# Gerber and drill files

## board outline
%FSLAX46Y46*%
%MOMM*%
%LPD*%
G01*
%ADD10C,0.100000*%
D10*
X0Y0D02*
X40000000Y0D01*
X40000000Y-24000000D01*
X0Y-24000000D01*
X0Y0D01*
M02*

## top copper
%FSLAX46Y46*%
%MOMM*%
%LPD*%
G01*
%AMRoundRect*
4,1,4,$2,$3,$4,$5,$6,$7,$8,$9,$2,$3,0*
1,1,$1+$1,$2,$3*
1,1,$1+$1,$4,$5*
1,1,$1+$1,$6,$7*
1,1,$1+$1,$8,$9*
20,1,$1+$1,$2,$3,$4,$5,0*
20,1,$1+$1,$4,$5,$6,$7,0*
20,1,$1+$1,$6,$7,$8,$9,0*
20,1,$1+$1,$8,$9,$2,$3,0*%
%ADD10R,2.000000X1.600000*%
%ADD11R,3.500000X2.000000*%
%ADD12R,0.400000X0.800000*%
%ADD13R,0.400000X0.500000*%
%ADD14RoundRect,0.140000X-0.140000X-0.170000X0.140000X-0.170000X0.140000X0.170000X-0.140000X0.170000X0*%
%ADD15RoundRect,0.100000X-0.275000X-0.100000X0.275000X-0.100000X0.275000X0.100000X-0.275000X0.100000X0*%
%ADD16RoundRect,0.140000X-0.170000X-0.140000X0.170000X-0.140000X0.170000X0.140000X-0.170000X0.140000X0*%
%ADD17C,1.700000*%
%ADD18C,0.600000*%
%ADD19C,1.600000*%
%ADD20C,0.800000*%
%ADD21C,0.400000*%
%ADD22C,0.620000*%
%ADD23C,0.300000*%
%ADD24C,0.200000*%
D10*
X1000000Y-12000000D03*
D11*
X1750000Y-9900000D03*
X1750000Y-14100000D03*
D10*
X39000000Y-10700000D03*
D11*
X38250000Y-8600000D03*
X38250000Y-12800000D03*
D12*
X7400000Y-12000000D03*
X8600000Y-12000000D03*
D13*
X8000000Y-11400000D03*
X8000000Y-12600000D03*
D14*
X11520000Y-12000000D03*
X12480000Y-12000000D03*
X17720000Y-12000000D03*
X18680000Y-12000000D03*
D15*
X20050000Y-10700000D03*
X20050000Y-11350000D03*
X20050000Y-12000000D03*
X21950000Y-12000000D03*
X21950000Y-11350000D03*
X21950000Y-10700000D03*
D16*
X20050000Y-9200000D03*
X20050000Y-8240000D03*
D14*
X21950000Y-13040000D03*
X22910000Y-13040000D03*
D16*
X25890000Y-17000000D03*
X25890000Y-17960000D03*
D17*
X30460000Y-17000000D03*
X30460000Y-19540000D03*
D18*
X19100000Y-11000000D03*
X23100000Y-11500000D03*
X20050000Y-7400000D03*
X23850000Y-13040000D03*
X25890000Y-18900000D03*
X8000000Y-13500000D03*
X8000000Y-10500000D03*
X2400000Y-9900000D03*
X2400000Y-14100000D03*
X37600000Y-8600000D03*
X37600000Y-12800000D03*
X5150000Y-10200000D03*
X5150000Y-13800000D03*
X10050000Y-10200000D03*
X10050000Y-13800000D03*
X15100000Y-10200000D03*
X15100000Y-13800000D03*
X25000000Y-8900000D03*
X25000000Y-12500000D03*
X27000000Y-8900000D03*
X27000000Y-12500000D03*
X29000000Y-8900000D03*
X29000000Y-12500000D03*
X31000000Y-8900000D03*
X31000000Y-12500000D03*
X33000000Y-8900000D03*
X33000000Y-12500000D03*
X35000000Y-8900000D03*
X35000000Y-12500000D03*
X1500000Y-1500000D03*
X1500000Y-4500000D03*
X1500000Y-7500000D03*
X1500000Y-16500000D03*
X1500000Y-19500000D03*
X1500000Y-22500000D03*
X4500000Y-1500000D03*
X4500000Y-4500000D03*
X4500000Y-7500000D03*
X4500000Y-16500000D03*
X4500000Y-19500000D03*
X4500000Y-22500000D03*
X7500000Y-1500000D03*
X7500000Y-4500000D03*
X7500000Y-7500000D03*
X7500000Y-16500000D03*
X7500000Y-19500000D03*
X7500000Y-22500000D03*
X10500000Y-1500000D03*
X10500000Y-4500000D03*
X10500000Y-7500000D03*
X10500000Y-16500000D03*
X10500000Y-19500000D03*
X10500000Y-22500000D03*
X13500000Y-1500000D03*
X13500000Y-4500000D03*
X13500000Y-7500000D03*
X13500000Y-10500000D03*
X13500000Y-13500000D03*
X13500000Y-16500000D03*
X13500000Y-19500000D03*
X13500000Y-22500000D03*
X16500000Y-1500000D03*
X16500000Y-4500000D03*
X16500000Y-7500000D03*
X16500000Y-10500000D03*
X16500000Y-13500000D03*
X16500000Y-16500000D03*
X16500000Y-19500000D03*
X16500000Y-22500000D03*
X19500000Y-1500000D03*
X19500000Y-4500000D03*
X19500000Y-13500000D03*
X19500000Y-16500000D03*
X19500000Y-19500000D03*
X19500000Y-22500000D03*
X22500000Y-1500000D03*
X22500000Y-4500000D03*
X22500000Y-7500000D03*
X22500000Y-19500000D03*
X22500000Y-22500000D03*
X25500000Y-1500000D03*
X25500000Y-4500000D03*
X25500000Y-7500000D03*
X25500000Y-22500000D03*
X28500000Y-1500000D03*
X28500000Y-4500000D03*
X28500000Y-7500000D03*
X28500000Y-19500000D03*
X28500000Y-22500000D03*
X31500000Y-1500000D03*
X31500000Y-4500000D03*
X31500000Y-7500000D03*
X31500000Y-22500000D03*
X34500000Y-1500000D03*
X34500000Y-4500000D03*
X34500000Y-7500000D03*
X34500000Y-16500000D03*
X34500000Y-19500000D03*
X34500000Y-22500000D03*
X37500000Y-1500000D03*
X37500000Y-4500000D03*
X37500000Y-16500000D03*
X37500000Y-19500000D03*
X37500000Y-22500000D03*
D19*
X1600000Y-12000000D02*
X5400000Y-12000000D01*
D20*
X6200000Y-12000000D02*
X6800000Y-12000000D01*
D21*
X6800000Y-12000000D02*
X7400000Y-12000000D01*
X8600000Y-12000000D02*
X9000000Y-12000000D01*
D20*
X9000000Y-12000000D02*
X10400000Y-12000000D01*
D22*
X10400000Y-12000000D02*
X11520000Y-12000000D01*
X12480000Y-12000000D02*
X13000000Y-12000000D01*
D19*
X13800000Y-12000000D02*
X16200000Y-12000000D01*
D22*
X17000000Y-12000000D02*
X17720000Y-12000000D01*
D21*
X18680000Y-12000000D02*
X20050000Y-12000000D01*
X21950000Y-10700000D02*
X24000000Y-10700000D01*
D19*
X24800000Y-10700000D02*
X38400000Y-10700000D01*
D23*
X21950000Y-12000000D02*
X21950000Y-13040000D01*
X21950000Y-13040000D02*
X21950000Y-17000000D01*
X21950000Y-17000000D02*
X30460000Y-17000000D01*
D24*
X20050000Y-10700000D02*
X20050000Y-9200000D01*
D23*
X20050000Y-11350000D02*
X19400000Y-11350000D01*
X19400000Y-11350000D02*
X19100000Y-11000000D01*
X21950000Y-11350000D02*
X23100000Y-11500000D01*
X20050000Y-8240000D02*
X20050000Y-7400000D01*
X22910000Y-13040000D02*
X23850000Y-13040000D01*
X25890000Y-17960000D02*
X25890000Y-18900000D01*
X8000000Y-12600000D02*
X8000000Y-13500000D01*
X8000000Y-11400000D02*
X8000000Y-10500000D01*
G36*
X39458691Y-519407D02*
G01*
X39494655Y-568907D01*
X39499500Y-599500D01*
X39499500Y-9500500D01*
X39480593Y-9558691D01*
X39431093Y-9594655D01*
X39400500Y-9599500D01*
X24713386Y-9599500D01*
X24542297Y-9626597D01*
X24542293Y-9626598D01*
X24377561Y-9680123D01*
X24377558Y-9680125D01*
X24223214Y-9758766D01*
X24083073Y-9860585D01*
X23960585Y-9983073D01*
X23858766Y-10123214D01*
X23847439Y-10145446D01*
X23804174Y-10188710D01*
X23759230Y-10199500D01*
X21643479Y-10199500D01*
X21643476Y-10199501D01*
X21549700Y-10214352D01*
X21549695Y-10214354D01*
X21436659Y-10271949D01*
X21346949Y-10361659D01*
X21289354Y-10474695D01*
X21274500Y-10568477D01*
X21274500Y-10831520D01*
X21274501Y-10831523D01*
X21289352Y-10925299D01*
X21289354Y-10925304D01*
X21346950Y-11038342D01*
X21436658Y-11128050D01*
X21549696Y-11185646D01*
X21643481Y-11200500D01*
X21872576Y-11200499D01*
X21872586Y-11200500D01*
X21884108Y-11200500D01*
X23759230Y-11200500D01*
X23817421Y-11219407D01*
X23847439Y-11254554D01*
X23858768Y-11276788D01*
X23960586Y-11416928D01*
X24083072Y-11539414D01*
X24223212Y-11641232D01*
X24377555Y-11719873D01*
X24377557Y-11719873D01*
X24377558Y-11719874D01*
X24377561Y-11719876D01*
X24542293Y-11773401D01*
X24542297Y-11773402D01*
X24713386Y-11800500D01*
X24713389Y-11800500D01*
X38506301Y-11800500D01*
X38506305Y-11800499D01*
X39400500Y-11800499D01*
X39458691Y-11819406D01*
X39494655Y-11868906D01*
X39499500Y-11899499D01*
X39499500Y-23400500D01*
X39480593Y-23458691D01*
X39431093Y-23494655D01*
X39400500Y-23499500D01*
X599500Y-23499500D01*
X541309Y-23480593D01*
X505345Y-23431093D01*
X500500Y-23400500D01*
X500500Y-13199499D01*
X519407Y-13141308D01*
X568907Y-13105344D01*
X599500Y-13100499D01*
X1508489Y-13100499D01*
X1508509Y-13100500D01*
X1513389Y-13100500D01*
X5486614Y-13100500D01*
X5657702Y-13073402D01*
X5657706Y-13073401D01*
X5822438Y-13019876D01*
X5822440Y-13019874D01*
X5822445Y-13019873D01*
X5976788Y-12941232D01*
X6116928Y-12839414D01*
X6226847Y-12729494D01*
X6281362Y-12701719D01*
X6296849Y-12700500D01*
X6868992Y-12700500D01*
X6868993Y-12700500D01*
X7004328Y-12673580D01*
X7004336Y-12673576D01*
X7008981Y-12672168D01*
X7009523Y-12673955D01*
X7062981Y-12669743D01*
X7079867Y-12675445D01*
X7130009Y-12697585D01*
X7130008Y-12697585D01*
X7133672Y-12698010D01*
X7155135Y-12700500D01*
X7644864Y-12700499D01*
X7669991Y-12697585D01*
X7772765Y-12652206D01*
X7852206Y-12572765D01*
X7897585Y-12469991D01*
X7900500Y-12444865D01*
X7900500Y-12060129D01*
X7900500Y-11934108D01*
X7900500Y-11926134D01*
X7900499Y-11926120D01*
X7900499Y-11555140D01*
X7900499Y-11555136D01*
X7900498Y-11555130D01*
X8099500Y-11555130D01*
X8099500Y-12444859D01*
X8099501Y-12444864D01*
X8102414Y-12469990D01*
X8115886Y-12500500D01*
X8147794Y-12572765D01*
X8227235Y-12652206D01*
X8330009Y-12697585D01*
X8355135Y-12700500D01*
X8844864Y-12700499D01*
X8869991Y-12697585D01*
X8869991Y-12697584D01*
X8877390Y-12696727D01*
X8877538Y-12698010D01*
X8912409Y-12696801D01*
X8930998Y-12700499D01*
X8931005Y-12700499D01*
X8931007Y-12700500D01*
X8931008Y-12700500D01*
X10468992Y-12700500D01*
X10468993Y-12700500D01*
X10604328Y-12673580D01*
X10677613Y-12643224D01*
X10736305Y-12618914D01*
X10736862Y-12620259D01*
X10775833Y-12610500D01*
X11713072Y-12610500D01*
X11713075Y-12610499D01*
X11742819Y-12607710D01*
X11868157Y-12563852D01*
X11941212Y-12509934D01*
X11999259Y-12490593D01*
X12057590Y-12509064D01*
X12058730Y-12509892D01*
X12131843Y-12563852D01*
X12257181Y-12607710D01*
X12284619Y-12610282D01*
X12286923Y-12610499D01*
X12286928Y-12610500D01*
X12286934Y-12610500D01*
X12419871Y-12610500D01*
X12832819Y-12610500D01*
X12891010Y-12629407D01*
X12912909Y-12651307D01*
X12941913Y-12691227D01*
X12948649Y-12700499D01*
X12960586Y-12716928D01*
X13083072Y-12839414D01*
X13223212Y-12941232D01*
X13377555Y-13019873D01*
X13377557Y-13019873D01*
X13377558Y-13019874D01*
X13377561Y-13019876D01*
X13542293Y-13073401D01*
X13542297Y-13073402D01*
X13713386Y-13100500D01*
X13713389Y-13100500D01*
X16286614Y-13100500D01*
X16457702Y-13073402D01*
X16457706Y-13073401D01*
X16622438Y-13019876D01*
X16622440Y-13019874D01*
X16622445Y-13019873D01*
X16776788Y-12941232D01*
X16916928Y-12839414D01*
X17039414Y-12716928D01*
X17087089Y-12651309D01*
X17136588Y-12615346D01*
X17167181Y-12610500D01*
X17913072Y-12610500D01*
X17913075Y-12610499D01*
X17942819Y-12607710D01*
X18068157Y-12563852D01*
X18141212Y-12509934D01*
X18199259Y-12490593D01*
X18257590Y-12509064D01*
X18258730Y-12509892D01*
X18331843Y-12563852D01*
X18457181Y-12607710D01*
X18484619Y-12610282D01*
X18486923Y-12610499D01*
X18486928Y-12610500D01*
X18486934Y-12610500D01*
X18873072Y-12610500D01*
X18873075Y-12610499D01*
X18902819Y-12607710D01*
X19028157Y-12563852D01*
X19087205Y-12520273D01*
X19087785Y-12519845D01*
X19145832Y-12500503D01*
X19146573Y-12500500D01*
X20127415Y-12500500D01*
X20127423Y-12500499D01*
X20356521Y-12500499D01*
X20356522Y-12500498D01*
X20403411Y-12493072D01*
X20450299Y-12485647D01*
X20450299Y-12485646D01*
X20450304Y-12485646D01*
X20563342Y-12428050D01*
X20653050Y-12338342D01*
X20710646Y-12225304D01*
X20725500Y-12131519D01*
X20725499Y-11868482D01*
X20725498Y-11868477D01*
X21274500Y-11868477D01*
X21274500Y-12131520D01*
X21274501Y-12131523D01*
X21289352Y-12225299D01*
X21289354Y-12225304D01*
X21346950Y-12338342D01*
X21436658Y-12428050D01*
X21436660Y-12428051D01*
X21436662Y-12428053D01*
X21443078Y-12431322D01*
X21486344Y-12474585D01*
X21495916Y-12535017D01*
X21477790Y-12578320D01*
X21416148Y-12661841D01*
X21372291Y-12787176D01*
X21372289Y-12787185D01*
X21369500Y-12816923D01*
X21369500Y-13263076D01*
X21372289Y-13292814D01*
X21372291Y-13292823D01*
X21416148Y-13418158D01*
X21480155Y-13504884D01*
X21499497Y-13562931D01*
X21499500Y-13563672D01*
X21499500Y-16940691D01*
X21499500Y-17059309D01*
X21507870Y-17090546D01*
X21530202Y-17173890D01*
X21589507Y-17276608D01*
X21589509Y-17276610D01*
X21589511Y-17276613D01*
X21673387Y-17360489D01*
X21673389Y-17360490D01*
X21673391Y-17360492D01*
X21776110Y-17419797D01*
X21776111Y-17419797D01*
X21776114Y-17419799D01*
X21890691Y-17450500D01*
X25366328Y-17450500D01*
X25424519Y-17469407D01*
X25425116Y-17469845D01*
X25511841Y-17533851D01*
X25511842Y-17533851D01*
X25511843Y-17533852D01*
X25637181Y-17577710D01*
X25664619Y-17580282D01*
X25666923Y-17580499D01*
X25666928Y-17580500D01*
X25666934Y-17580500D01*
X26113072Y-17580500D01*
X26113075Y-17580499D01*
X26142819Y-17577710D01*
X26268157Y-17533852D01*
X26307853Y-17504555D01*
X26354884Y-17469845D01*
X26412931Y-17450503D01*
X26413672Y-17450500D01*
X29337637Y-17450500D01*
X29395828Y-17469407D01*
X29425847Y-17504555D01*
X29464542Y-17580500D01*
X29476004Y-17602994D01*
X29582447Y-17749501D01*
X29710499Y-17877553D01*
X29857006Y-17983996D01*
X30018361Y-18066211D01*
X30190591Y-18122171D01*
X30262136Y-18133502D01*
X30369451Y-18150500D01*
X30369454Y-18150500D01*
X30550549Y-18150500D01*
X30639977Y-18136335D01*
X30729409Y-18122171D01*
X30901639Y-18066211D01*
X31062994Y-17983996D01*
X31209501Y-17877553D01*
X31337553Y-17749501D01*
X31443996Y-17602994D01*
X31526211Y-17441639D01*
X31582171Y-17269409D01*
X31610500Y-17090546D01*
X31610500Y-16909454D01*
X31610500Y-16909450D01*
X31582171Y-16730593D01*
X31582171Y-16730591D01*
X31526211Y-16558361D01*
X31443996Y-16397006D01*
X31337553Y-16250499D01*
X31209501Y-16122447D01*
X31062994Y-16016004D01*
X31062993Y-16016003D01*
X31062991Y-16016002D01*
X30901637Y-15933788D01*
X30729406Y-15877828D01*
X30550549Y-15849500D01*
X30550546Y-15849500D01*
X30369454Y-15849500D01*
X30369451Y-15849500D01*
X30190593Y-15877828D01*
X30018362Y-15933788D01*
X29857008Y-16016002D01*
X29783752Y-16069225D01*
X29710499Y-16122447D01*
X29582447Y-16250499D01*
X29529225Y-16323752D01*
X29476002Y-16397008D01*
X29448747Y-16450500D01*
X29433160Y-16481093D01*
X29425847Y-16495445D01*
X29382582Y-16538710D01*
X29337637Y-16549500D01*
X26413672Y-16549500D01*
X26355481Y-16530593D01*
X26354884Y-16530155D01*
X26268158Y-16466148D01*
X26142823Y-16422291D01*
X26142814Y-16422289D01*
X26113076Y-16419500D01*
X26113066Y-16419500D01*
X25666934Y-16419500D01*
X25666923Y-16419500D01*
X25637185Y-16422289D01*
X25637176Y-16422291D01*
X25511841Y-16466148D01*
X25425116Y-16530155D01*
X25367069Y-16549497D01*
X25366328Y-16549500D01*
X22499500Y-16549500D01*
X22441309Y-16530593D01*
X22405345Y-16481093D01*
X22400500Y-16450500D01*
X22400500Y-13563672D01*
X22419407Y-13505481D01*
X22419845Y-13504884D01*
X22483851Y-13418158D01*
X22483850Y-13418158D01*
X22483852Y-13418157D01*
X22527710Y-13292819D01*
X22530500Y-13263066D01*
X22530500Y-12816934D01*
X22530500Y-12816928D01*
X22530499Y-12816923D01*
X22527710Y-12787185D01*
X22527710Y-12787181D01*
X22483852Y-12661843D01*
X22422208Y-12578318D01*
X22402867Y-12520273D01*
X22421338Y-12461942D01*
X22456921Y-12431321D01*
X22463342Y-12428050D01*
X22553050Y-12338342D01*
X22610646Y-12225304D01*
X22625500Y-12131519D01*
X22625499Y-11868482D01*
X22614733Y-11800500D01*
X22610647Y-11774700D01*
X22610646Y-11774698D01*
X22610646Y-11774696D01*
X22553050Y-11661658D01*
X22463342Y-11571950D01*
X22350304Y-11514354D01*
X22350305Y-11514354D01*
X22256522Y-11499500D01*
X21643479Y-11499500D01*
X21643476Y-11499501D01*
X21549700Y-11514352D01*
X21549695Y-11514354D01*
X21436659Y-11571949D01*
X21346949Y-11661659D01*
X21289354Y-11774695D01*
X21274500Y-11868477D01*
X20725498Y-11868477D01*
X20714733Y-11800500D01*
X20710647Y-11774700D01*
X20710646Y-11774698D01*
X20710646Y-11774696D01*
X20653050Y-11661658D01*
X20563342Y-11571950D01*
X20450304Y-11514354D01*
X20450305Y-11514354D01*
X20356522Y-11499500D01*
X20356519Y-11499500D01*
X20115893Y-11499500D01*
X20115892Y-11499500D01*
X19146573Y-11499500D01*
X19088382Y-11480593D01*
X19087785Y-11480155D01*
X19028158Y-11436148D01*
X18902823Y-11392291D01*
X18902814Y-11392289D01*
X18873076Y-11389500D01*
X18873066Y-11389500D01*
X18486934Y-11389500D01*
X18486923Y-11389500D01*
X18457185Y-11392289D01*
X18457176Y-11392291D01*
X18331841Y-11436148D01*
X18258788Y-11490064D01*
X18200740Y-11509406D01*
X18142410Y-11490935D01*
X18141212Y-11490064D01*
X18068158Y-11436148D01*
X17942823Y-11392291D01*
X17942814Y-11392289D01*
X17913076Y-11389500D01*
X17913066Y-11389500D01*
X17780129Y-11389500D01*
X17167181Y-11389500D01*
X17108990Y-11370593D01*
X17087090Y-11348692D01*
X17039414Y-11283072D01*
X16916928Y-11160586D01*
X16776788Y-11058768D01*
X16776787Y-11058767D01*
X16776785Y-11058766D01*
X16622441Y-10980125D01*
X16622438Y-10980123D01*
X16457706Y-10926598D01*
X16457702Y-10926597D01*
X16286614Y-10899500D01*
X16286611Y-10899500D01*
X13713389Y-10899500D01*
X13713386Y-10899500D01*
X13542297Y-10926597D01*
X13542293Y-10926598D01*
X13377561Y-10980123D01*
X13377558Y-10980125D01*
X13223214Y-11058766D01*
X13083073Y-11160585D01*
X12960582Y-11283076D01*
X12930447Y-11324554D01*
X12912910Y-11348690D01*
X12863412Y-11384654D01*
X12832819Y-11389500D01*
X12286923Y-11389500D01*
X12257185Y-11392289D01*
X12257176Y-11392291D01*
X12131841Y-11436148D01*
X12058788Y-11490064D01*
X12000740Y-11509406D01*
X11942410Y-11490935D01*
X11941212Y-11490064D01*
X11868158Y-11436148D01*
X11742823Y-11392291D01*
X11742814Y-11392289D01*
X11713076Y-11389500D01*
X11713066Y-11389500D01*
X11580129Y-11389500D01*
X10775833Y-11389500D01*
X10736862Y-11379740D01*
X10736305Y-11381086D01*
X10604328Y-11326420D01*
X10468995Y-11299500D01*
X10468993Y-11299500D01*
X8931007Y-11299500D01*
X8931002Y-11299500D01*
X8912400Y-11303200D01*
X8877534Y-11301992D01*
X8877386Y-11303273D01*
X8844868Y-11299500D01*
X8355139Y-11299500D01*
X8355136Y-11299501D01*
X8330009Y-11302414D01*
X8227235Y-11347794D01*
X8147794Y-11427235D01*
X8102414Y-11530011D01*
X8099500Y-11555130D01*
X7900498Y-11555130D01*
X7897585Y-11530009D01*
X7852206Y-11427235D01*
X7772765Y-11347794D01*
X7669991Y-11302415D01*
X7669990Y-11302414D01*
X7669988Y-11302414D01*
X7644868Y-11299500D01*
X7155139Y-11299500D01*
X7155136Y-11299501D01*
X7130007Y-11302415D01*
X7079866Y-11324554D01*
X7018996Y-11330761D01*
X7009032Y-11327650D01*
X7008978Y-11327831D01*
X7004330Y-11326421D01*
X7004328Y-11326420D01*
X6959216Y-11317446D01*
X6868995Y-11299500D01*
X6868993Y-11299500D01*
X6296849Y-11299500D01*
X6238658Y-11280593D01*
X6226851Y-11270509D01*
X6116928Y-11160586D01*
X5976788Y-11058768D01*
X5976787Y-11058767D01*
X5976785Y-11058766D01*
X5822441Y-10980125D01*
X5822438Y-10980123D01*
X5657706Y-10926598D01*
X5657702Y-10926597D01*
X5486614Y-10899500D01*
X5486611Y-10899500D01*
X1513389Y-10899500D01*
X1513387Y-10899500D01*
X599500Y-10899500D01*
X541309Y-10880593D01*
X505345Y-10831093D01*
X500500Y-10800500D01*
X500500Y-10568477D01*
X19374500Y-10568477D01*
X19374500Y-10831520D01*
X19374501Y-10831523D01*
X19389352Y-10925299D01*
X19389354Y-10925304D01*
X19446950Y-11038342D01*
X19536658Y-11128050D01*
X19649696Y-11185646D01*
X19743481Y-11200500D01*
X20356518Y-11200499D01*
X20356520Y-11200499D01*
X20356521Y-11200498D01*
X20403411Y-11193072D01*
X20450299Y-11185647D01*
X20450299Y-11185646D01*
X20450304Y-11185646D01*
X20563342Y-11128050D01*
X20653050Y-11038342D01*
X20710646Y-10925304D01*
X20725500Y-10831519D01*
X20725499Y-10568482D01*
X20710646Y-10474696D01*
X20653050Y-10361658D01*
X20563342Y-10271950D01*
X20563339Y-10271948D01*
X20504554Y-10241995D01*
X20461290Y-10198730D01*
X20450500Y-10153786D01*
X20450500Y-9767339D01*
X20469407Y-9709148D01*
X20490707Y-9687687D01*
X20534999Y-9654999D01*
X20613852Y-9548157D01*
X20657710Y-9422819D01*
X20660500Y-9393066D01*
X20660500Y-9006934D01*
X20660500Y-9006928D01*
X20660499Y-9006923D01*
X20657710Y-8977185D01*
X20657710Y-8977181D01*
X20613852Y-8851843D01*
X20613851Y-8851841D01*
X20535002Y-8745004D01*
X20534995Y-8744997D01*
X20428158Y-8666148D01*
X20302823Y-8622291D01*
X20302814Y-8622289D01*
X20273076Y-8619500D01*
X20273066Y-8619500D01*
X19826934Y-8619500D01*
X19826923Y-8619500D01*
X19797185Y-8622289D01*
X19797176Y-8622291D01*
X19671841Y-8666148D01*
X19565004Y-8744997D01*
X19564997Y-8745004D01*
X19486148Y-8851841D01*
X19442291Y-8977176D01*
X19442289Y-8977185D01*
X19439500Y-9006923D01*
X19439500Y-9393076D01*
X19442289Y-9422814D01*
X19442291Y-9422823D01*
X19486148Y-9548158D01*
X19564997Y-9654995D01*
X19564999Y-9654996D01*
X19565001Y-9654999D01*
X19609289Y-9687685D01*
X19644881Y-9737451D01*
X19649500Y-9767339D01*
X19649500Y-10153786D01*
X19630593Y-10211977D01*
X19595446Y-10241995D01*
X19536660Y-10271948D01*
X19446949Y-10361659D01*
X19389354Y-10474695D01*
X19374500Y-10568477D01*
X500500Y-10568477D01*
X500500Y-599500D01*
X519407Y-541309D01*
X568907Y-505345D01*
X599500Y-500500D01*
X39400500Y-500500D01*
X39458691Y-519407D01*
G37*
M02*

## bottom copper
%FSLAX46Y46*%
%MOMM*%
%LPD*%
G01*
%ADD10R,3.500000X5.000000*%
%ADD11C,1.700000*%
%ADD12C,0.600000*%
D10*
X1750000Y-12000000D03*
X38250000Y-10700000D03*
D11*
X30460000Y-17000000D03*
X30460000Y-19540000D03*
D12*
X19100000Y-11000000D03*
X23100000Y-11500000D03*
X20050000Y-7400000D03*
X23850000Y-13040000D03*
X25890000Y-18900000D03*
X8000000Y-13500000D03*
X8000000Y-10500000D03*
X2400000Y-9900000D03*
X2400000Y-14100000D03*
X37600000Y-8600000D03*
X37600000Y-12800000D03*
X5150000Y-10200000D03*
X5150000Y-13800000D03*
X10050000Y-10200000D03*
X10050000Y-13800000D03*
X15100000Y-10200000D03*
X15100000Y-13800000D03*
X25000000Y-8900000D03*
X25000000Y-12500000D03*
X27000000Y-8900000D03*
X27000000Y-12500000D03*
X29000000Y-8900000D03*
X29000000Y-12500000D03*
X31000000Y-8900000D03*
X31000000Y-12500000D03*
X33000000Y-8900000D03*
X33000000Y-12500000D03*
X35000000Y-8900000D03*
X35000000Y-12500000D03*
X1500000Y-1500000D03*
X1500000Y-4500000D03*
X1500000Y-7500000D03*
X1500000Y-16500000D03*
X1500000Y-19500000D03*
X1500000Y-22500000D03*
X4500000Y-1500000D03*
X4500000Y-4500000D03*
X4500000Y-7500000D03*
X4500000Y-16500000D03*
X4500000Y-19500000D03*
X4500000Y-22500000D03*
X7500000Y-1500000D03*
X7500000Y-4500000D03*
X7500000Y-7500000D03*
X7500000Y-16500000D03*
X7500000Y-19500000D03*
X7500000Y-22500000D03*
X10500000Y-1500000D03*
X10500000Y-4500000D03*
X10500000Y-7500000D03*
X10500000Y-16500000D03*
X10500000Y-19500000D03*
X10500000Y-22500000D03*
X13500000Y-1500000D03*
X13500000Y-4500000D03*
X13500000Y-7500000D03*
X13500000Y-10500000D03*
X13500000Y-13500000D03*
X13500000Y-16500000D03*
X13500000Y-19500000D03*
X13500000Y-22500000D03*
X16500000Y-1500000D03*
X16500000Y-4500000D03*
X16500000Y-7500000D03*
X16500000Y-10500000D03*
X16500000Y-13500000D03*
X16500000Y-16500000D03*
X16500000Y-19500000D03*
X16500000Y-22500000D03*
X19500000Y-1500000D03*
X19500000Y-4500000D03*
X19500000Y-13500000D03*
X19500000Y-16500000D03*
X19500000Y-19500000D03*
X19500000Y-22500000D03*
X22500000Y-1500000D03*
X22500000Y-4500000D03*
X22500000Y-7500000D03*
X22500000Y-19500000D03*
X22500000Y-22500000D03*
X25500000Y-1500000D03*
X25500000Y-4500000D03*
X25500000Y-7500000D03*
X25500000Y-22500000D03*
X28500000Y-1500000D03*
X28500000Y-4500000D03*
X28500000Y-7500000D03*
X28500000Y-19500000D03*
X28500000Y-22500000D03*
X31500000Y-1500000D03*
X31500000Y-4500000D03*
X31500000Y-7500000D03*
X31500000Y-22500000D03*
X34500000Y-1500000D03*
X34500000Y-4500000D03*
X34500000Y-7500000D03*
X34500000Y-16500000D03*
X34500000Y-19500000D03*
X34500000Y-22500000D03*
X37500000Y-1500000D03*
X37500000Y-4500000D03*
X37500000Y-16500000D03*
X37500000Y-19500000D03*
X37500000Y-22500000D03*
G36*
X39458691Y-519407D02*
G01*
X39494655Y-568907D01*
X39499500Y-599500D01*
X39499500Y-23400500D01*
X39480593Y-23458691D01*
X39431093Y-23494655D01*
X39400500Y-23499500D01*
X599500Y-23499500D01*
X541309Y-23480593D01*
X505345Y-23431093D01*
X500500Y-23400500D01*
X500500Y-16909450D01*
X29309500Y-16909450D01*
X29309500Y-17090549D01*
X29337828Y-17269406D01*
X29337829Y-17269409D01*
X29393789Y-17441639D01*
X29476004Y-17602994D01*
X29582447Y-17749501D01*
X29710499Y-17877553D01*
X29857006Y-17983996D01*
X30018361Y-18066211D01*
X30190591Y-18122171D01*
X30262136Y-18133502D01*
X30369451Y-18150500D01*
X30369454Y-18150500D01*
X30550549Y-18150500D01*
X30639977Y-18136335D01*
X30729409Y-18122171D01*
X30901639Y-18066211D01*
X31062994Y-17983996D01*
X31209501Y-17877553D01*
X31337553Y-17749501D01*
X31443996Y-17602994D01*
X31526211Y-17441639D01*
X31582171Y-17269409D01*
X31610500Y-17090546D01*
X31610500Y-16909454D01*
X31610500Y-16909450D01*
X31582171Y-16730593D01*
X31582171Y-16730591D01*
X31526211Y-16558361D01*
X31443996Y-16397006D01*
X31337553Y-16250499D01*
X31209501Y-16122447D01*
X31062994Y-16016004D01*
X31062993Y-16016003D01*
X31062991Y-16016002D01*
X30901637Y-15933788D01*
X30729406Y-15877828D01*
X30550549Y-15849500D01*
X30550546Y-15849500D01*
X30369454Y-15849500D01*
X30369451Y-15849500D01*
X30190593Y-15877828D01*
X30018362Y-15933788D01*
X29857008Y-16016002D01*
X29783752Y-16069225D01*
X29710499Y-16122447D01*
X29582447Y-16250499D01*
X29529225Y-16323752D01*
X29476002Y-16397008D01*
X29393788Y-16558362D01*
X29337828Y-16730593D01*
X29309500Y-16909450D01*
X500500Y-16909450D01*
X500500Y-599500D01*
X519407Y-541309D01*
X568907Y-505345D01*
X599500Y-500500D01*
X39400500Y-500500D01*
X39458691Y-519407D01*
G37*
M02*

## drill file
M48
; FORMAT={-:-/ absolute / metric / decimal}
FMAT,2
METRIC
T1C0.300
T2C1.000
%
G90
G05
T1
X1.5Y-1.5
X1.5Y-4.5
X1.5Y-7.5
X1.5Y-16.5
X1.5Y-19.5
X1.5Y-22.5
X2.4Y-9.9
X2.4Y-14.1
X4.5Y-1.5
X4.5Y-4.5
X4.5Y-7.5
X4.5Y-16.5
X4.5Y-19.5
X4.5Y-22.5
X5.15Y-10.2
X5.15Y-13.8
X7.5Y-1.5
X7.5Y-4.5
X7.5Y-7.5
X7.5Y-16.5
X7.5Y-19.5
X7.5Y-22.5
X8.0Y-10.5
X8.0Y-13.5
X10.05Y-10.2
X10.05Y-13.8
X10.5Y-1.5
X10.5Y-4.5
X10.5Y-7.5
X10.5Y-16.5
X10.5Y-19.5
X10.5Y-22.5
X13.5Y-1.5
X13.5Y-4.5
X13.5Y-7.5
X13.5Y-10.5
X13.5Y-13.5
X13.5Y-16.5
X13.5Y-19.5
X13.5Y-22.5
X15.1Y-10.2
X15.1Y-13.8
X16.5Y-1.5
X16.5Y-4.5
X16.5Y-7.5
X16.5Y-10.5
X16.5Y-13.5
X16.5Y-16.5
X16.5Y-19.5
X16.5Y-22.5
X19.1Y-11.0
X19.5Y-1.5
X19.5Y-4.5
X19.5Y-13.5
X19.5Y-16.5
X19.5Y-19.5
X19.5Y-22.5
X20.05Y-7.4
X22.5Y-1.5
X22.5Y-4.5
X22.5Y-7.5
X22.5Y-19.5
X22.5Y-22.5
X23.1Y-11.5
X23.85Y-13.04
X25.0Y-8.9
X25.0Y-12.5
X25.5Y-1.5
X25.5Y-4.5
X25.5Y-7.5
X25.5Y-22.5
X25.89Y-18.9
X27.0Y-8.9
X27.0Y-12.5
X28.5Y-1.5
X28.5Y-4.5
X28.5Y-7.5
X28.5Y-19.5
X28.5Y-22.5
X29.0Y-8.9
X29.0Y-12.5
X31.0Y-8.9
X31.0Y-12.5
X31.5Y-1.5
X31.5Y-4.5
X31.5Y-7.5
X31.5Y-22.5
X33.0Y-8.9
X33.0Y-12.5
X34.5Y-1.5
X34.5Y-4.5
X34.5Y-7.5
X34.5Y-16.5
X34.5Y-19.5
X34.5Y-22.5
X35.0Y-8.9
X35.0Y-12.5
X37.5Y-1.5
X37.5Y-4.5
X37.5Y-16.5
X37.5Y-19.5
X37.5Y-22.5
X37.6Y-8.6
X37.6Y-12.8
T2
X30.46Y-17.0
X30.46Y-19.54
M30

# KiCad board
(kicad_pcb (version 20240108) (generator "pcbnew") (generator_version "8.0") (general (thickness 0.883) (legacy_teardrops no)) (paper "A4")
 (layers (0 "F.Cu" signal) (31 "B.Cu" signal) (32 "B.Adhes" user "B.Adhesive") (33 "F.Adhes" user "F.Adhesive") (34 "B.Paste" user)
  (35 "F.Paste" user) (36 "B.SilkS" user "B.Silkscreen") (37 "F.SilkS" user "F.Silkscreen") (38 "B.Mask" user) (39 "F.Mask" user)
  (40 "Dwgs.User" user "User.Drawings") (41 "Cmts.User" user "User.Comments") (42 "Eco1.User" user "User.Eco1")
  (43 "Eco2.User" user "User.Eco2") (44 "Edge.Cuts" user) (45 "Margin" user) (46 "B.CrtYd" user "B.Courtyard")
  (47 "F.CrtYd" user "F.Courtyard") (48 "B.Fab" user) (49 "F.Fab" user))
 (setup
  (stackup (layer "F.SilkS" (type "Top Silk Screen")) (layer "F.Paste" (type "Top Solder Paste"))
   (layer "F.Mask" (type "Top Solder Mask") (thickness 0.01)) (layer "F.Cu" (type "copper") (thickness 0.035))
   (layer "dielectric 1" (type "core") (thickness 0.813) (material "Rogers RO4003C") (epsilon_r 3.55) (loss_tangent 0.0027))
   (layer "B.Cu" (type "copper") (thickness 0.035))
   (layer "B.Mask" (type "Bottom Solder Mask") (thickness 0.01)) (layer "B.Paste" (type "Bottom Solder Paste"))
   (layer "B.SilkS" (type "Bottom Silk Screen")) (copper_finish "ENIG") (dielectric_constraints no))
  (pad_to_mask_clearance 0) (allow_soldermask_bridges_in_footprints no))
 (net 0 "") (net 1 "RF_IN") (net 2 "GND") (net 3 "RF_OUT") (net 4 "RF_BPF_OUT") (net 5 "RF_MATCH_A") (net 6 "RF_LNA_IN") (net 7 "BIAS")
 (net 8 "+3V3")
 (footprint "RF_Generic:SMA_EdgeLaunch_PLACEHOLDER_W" (layer "F.Cu") (at 0 12)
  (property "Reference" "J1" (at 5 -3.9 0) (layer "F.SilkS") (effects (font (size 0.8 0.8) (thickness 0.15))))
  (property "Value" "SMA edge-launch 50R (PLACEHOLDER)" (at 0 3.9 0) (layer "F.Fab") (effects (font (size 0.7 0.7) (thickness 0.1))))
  (pad "1" smd rect (at 1 0) (size 2 1.6) (layers "F.Cu" "F.Paste" "F.Mask") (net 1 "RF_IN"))
  (pad "2" smd rect (at 1.75 -2.1) (size 3.5 2) (layers "F.Cu" "F.Paste" "F.Mask") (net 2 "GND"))
  (pad "3" smd rect (at 1.75 2.1) (size 3.5 2) (layers "F.Cu" "F.Paste" "F.Mask") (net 2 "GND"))
  (pad "4" smd rect (at 1.75 0) (size 3.5 5) (layers "B.Cu" "B.Paste" "B.Mask") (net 2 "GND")))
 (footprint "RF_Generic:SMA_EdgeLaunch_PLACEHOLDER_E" (layer "F.Cu") (at 40 10.7)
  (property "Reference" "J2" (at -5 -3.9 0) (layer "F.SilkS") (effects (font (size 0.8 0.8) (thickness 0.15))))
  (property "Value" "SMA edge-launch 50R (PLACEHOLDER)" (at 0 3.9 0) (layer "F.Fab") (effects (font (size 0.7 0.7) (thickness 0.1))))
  (pad "1" smd rect (at -1 0) (size 2 1.6) (layers "F.Cu" "F.Paste" "F.Mask") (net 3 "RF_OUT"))
  (pad "2" smd rect (at -1.75 -2.1) (size 3.5 2) (layers "F.Cu" "F.Paste" "F.Mask") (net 2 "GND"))
  (pad "3" smd rect (at -1.75 2.1) (size 3.5 2) (layers "F.Cu" "F.Paste" "F.Mask") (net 2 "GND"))
  (pad "4" smd rect (at -1.75 0) (size 3.5 5) (layers "B.Cu" "B.Paste" "B.Mask") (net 2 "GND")))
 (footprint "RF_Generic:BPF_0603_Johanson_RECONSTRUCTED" (layer "F.Cu") (at 8 12)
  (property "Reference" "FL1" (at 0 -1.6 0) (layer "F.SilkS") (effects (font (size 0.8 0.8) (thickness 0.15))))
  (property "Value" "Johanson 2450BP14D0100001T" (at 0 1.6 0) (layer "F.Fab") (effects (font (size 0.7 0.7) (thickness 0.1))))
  (pad "2" smd rect (at -0.6 0) (size 0.4 0.8) (layers "F.Cu" "F.Paste" "F.Mask") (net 1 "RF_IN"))
  (pad "4" smd rect (at 0.6 0) (size 0.4 0.8) (layers "F.Cu" "F.Paste" "F.Mask") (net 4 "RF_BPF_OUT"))
  (pad "1" smd rect (at 0 -0.6) (size 0.4 0.5) (layers "F.Cu" "F.Paste" "F.Mask") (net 2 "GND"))
  (pad "3" smd rect (at 0 0.6) (size 0.4 0.5) (layers "F.Cu" "F.Paste" "F.Mask") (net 2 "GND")))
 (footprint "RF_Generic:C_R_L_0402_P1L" (layer "F.Cu") (at 12 12)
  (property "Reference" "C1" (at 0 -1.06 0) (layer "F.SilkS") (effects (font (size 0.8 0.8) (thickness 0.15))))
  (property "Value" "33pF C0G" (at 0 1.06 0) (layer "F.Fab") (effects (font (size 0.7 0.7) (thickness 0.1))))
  (pad "1" smd roundrect (at -0.48 0) (size 0.56 0.62) (layers "F.Cu" "F.Paste" "F.Mask") (roundrect_rratio 0.25) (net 4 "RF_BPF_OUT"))
  (pad "2" smd roundrect (at 0.48 0) (size 0.56 0.62) (layers "F.Cu" "F.Paste" "F.Mask") (roundrect_rratio 0.25) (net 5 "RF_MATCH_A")))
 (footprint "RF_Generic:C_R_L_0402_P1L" (layer "F.Cu") (at 18.2 12)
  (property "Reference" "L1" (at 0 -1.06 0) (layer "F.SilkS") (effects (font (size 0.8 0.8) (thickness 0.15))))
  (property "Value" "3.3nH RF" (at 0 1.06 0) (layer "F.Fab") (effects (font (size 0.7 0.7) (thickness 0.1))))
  (pad "1" smd roundrect (at -0.48 0) (size 0.56 0.62) (layers "F.Cu" "F.Paste" "F.Mask") (roundrect_rratio 0.25) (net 5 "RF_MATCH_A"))
  (pad "2" smd roundrect (at 0.48 0) (size 0.56 0.62) (layers "F.Cu" "F.Paste" "F.Mask") (roundrect_rratio 0.25) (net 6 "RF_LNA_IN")))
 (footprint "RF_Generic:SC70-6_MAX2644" (layer "F.Cu") (at 21 11.35)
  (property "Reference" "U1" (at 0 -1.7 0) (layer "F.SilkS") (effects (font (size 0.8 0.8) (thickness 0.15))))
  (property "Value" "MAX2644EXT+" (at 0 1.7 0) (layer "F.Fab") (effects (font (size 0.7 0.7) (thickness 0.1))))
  (pad "1" smd roundrect (at -0.95 -0.65) (size 0.75 0.4) (layers "F.Cu" "F.Paste" "F.Mask") (roundrect_rratio 0.25) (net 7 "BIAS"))
  (pad "2" smd roundrect (at -0.95 0) (size 0.75 0.4) (layers "F.Cu" "F.Paste" "F.Mask") (roundrect_rratio 0.25) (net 2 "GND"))
  (pad "3" smd roundrect (at -0.95 0.65) (size 0.75 0.4) (layers "F.Cu" "F.Paste" "F.Mask") (roundrect_rratio 0.25) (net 6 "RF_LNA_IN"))
  (pad "4" smd roundrect (at 0.95 0.65) (size 0.75 0.4) (layers "F.Cu" "F.Paste" "F.Mask") (roundrect_rratio 0.25) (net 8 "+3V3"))
  (pad "5" smd roundrect (at 0.95 0) (size 0.75 0.4) (layers "F.Cu" "F.Paste" "F.Mask") (roundrect_rratio 0.25) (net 2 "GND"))
  (pad "6" smd roundrect (at 0.95 -0.65) (size 0.75 0.4) (layers "F.Cu" "F.Paste" "F.Mask") (roundrect_rratio 0.25) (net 3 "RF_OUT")))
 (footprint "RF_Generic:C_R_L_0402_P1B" (layer "F.Cu") (at 20.05 8.72)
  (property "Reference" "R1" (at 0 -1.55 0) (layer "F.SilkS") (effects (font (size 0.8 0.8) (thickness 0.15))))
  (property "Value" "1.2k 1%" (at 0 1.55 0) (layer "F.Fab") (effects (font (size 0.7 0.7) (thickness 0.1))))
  (pad "1" smd roundrect (at 0 0.48) (size 0.62 0.56) (layers "F.Cu" "F.Paste" "F.Mask") (roundrect_rratio 0.25) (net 7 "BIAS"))
  (pad "2" smd roundrect (at 0 -0.48) (size 0.62 0.56) (layers "F.Cu" "F.Paste" "F.Mask") (roundrect_rratio 0.25) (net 2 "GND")))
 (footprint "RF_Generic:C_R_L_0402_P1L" (layer "F.Cu") (at 22.43 13.04)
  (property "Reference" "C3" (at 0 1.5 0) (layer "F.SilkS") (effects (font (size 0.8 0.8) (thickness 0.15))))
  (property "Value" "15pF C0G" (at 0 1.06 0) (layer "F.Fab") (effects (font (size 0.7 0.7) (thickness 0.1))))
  (pad "1" smd roundrect (at -0.48 0) (size 0.56 0.62) (layers "F.Cu" "F.Paste" "F.Mask") (roundrect_rratio 0.25) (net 8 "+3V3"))
  (pad "2" smd roundrect (at 0.48 0) (size 0.56 0.62) (layers "F.Cu" "F.Paste" "F.Mask") (roundrect_rratio 0.25) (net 2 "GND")))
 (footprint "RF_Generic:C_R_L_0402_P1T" (layer "F.Cu") (at 25.89 17.48)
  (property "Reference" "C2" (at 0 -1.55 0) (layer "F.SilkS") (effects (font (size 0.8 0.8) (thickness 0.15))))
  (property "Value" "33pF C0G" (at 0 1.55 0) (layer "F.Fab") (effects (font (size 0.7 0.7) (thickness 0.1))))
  (pad "1" smd roundrect (at 0 -0.48) (size 0.62 0.56) (layers "F.Cu" "F.Paste" "F.Mask") (roundrect_rratio 0.25) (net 8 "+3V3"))
  (pad "2" smd roundrect (at 0 0.48) (size 0.62 0.56) (layers "F.Cu" "F.Paste" "F.Mask") (roundrect_rratio 0.25) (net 2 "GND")))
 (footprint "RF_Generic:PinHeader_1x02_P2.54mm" (layer "F.Cu") (at 30.46 17)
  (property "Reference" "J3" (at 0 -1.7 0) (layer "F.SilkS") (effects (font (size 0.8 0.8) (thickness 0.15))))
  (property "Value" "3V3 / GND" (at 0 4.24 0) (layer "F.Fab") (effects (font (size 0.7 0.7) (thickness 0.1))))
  (pad "1" thru_hole circle (at 0 0) (size 1.7 1.7) (drill 1) (layers "*.Cu" "*.Mask") (remove_unused_layers no) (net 8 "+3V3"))
  (pad "2" thru_hole circle (at 0 2.54) (size 1.7 1.7) (drill 1) (layers "*.Cu" "*.Mask") (remove_unused_layers no) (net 2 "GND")))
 (segment (start 1.6 12) (end 5.4 12) (width 1.6) (layer "F.Cu") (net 1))
 (segment (start 6.2 12) (end 6.8 12) (width 0.8) (layer "F.Cu") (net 1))
 (segment (start 6.8 12) (end 7.4 12) (width 0.4) (layer "F.Cu") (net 1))
 (segment (start 8.6 12) (end 9 12) (width 0.4) (layer "F.Cu") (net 4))
 (segment (start 9 12) (end 10.4 12) (width 0.8) (layer "F.Cu") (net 4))
 (segment (start 10.4 12) (end 11.52 12) (width 0.62) (layer "F.Cu") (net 4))
 (segment (start 12.48 12) (end 13 12) (width 0.62) (layer "F.Cu") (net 5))
 (segment (start 13.8 12) (end 16.2 12) (width 1.6) (layer "F.Cu") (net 5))
 (segment (start 17 12) (end 17.72 12) (width 0.62) (layer "F.Cu") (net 5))
 (segment (start 18.68 12) (end 20.05 12) (width 0.4) (layer "F.Cu") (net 6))
 (segment (start 21.95 10.7) (end 24 10.7) (width 0.4) (layer "F.Cu") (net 3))
 (segment (start 24.8 10.7) (end 38.4 10.7) (width 1.6) (layer "F.Cu") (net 3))
 (segment (start 21.95 12) (end 21.95 13.04) (width 0.3) (layer "F.Cu") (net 8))
 (segment (start 21.95 13.04) (end 21.95 17) (width 0.3) (layer "F.Cu") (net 8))
 (segment (start 21.95 17) (end 30.46 17) (width 0.3) (layer "F.Cu") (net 8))
 (segment (start 20.05 10.7) (end 20.05 9.2) (width 0.2) (layer "F.Cu") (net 7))
 (segment (start 20.05 11.35) (end 19.4 11.35) (width 0.3) (layer "F.Cu") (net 2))
 (segment (start 19.4 11.35) (end 19.1 11) (width 0.3) (layer "F.Cu") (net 2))
 (segment (start 21.95 11.35) (end 23.1 11.5) (width 0.3) (layer "F.Cu") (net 2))
 (segment (start 20.05 8.24) (end 20.05 7.4) (width 0.3) (layer "F.Cu") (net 2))
 (segment (start 22.91 13.04) (end 23.85 13.04) (width 0.3) (layer "F.Cu") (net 2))
 (segment (start 25.89 17.96) (end 25.89 18.9) (width 0.3) (layer "F.Cu") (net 2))
 (segment (start 8 12.6) (end 8 13.5) (width 0.3) (layer "F.Cu") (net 2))
 (segment (start 8 11.4) (end 8 10.5) (width 0.3) (layer "F.Cu") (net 2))
 (via (at 19.1 11) (size 0.6) (drill 0.3) (layers "F.Cu" "B.Cu") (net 2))
 (via (at 23.1 11.5) (size 0.6) (drill 0.3) (layers "F.Cu" "B.Cu") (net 2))
 (via (at 20.05 7.4) (size 0.6) (drill 0.3) (layers "F.Cu" "B.Cu") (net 2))
 (via (at 23.85 13.04) (size 0.6) (drill 0.3) (layers "F.Cu" "B.Cu") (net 2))
 (via (at 25.89 18.9) (size 0.6) (drill 0.3) (layers "F.Cu" "B.Cu") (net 2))
 (via (at 8 13.5) (size 0.6) (drill 0.3) (layers "F.Cu" "B.Cu") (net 2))
 (via (at 8 10.5) (size 0.6) (drill 0.3) (layers "F.Cu" "B.Cu") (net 2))
 (via (at 2.4 9.9) (size 0.6) (drill 0.3) (layers "F.Cu" "B.Cu") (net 2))
 (via (at 2.4 14.1) (size 0.6) (drill 0.3) (layers "F.Cu" "B.Cu") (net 2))
 (via (at 37.6 8.6) (size 0.6) (drill 0.3) (layers "F.Cu" "B.Cu") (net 2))
 (via (at 37.6 12.8) (size 0.6) (drill 0.3) (layers "F.Cu" "B.Cu") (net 2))
 (via (at 5.15 10.2) (size 0.6) (drill 0.3) (layers "F.Cu" "B.Cu") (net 2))
 (via (at 5.15 13.8) (size 0.6) (drill 0.3) (layers "F.Cu" "B.Cu") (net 2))
 (via (at 10.05 10.2) (size 0.6) (drill 0.3) (layers "F.Cu" "B.Cu") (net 2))
 (via (at 10.05 13.8) (size 0.6) (drill 0.3) (layers "F.Cu" "B.Cu") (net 2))
 (via (at 15.1 10.2) (size 0.6) (drill 0.3) (layers "F.Cu" "B.Cu") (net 2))
 (via (at 15.1 13.8) (size 0.6) (drill 0.3) (layers "F.Cu" "B.Cu") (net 2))
 (via (at 25 8.9) (size 0.6) (drill 0.3) (layers "F.Cu" "B.Cu") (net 2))
 (via (at 25 12.5) (size 0.6) (drill 0.3) (layers "F.Cu" "B.Cu") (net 2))
 (via (at 27 8.9) (size 0.6) (drill 0.3) (layers "F.Cu" "B.Cu") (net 2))
 (via (at 27 12.5) (size 0.6) (drill 0.3) (layers "F.Cu" "B.Cu") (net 2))
 (via (at 29 8.9) (size 0.6) (drill 0.3) (layers "F.Cu" "B.Cu") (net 2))
 (via (at 29 12.5) (size 0.6) (drill 0.3) (layers "F.Cu" "B.Cu") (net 2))
 (via (at 31 8.9) (size 0.6) (drill 0.3) (layers "F.Cu" "B.Cu") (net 2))
 (via (at 31 12.5) (size 0.6) (drill 0.3) (layers "F.Cu" "B.Cu") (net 2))
 (via (at 33 8.9) (size 0.6) (drill 0.3) (layers "F.Cu" "B.Cu") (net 2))
 (via (at 33 12.5) (size 0.6) (drill 0.3) (layers "F.Cu" "B.Cu") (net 2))
 (via (at 35 8.9) (size 0.6) (drill 0.3) (layers "F.Cu" "B.Cu") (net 2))
 (via (at 35 12.5) (size 0.6) (drill 0.3) (layers "F.Cu" "B.Cu") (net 2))
 (via (at 1.5 1.5) (size 0.6) (drill 0.3) (layers "F.Cu" "B.Cu") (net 2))
 (via (at 1.5 4.5) (size 0.6) (drill 0.3) (layers "F.Cu" "B.Cu") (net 2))
 (via (at 1.5 7.5) (size 0.6) (drill 0.3) (layers "F.Cu" "B.Cu") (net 2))
 (via (at 1.5 16.5) (size 0.6) (drill 0.3) (layers "F.Cu" "B.Cu") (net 2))
 (via (at 1.5 19.5) (size 0.6) (drill 0.3) (layers "F.Cu" "B.Cu") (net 2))
 (via (at 1.5 22.5) (size 0.6) (drill 0.3) (layers "F.Cu" "B.Cu") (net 2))
 (via (at 4.5 1.5) (size 0.6) (drill 0.3) (layers "F.Cu" "B.Cu") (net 2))
 (via (at 4.5 4.5) (size 0.6) (drill 0.3) (layers "F.Cu" "B.Cu") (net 2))
 (via (at 4.5 7.5) (size 0.6) (drill 0.3) (layers "F.Cu" "B.Cu") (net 2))
 (via (at 4.5 16.5) (size 0.6) (drill 0.3) (layers "F.Cu" "B.Cu") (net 2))
 (via (at 4.5 19.5) (size 0.6) (drill 0.3) (layers "F.Cu" "B.Cu") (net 2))
 (via (at 4.5 22.5) (size 0.6) (drill 0.3) (layers "F.Cu" "B.Cu") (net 2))
 (via (at 7.5 1.5) (size 0.6) (drill 0.3) (layers "F.Cu" "B.Cu") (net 2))
 (via (at 7.5 4.5) (size 0.6) (drill 0.3) (layers "F.Cu" "B.Cu") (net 2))
 (via (at 7.5 7.5) (size 0.6) (drill 0.3) (layers "F.Cu" "B.Cu") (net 2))
 (via (at 7.5 16.5) (size 0.6) (drill 0.3) (layers "F.Cu" "B.Cu") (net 2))
 (via (at 7.5 19.5) (size 0.6) (drill 0.3) (layers "F.Cu" "B.Cu") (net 2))
 (via (at 7.5 22.5) (size 0.6) (drill 0.3) (layers "F.Cu" "B.Cu") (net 2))
 (via (at 10.5 1.5) (size 0.6) (drill 0.3) (layers "F.Cu" "B.Cu") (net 2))
 (via (at 10.5 4.5) (size 0.6) (drill 0.3) (layers "F.Cu" "B.Cu") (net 2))
 (via (at 10.5 7.5) (size 0.6) (drill 0.3) (layers "F.Cu" "B.Cu") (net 2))
 (via (at 10.5 16.5) (size 0.6) (drill 0.3) (layers "F.Cu" "B.Cu") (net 2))
 (via (at 10.5 19.5) (size 0.6) (drill 0.3) (layers "F.Cu" "B.Cu") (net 2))
 (via (at 10.5 22.5) (size 0.6) (drill 0.3) (layers "F.Cu" "B.Cu") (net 2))
 (via (at 13.5 1.5) (size 0.6) (drill 0.3) (layers "F.Cu" "B.Cu") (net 2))
 (via (at 13.5 4.5) (size 0.6) (drill 0.3) (layers "F.Cu" "B.Cu") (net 2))
 (via (at 13.5 7.5) (size 0.6) (drill 0.3) (layers "F.Cu" "B.Cu") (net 2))
 (via (at 13.5 10.5) (size 0.6) (drill 0.3) (layers "F.Cu" "B.Cu") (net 2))
 (via (at 13.5 13.5) (size 0.6) (drill 0.3) (layers "F.Cu" "B.Cu") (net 2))
 (via (at 13.5 16.5) (size 0.6) (drill 0.3) (layers "F.Cu" "B.Cu") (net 2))
 (via (at 13.5 19.5) (size 0.6) (drill 0.3) (layers "F.Cu" "B.Cu") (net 2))
 (via (at 13.5 22.5) (size 0.6) (drill 0.3) (layers "F.Cu" "B.Cu") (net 2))
 (via (at 16.5 1.5) (size 0.6) (drill 0.3) (layers "F.Cu" "B.Cu") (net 2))
 (via (at 16.5 4.5) (size 0.6) (drill 0.3) (layers "F.Cu" "B.Cu") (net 2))
 (via (at 16.5 7.5) (size 0.6) (drill 0.3) (layers "F.Cu" "B.Cu") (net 2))
 (via (at 16.5 10.5) (size 0.6) (drill 0.3) (layers "F.Cu" "B.Cu") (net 2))
 (via (at 16.5 13.5) (size 0.6) (drill 0.3) (layers "F.Cu" "B.Cu") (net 2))
 (via (at 16.5 16.5) (size 0.6) (drill 0.3) (layers "F.Cu" "B.Cu") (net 2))
 (via (at 16.5 19.5) (size 0.6) (drill 0.3) (layers "F.Cu" "B.Cu") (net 2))
 (via (at 16.5 22.5) (size 0.6) (drill 0.3) (layers "F.Cu" "B.Cu") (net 2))
 (via (at 19.5 1.5) (size 0.6) (drill 0.3) (layers "F.Cu" "B.Cu") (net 2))
 (via (at 19.5 4.5) (size 0.6) (drill 0.3) (layers "F.Cu" "B.Cu") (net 2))
 (via (at 19.5 13.5) (size 0.6) (drill 0.3) (layers "F.Cu" "B.Cu") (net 2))
 (via (at 19.5 16.5) (size 0.6) (drill 0.3) (layers "F.Cu" "B.Cu") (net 2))
 (via (at 19.5 19.5) (size 0.6) (drill 0.3) (layers "F.Cu" "B.Cu") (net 2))
 (via (at 19.5 22.5) (size 0.6) (drill 0.3) (layers "F.Cu" "B.Cu") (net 2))
 (via (at 22.5 1.5) (size 0.6) (drill 0.3) (layers "F.Cu" "B.Cu") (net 2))
 (via (at 22.5 4.5) (size 0.6) (drill 0.3) (layers "F.Cu" "B.Cu") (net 2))
 (via (at 22.5 7.5) (size 0.6) (drill 0.3) (layers "F.Cu" "B.Cu") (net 2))
 (via (at 22.5 19.5) (size 0.6) (drill 0.3) (layers "F.Cu" "B.Cu") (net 2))
 (via (at 22.5 22.5) (size 0.6) (drill 0.3) (layers "F.Cu" "B.Cu") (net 2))
 (via (at 25.5 1.5) (size 0.6) (drill 0.3) (layers "F.Cu" "B.Cu") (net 2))
 (via (at 25.5 4.5) (size 0.6) (drill 0.3) (layers "F.Cu" "B.Cu") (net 2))
 (via (at 25.5 7.5) (size 0.6) (drill 0.3) (layers "F.Cu" "B.Cu") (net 2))
 (via (at 25.5 22.5) (size 0.6) (drill 0.3) (layers "F.Cu" "B.Cu") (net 2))
 (via (at 28.5 1.5) (size 0.6) (drill 0.3) (layers "F.Cu" "B.Cu") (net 2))
 (via (at 28.5 4.5) (size 0.6) (drill 0.3) (layers "F.Cu" "B.Cu") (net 2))
 (via (at 28.5 7.5) (size 0.6) (drill 0.3) (layers "F.Cu" "B.Cu") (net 2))
 (via (at 28.5 19.5) (size 0.6) (drill 0.3) (layers "F.Cu" "B.Cu") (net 2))
 (via (at 28.5 22.5) (size 0.6) (drill 0.3) (layers "F.Cu" "B.Cu") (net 2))
 (via (at 31.5 1.5) (size 0.6) (drill 0.3) (layers "F.Cu" "B.Cu") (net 2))
 (via (at 31.5 4.5) (size 0.6) (drill 0.3) (layers "F.Cu" "B.Cu") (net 2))
 (via (at 31.5 7.5) (size 0.6) (drill 0.3) (layers "F.Cu" "B.Cu") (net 2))
 (via (at 31.5 22.5) (size 0.6) (drill 0.3) (layers "F.Cu" "B.Cu") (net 2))
 (via (at 34.5 1.5) (size 0.6) (drill 0.3) (layers "F.Cu" "B.Cu") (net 2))
 (via (at 34.5 4.5) (size 0.6) (drill 0.3) (layers "F.Cu" "B.Cu") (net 2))
 (via (at 34.5 7.5) (size 0.6) (drill 0.3) (layers "F.Cu" "B.Cu") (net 2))
 (via (at 34.5 16.5) (size 0.6) (drill 0.3) (layers "F.Cu" "B.Cu") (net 2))
 (via (at 34.5 19.5) (size 0.6) (drill 0.3) (layers "F.Cu" "B.Cu") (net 2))
 (via (at 34.5 22.5) (size 0.6) (drill 0.3) (layers "F.Cu" "B.Cu") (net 2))
 (via (at 37.5 1.5) (size 0.6) (drill 0.3) (layers "F.Cu" "B.Cu") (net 2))
 (via (at 37.5 4.5) (size 0.6) (drill 0.3) (layers "F.Cu" "B.Cu") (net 2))
 (via (at 37.5 16.5) (size 0.6) (drill 0.3) (layers "F.Cu" "B.Cu") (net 2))
 (via (at 37.5 19.5) (size 0.6) (drill 0.3) (layers "F.Cu" "B.Cu") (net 2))
 (via (at 37.5 22.5) (size 0.6) (drill 0.3) (layers "F.Cu" "B.Cu") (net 2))
 (gr_rect (start 0 0) (end 40 24) (stroke (width 0.1) (type default)) (fill none) (layer "Edge.Cuts"))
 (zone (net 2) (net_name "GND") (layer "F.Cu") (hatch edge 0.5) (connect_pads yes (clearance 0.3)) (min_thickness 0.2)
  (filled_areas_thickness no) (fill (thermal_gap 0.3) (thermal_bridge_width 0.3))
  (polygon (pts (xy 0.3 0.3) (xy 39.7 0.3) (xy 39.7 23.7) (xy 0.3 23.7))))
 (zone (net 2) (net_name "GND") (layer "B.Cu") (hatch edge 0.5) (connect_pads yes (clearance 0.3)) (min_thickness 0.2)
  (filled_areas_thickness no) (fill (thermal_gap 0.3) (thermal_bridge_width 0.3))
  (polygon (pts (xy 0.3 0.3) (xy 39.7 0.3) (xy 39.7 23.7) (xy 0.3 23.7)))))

